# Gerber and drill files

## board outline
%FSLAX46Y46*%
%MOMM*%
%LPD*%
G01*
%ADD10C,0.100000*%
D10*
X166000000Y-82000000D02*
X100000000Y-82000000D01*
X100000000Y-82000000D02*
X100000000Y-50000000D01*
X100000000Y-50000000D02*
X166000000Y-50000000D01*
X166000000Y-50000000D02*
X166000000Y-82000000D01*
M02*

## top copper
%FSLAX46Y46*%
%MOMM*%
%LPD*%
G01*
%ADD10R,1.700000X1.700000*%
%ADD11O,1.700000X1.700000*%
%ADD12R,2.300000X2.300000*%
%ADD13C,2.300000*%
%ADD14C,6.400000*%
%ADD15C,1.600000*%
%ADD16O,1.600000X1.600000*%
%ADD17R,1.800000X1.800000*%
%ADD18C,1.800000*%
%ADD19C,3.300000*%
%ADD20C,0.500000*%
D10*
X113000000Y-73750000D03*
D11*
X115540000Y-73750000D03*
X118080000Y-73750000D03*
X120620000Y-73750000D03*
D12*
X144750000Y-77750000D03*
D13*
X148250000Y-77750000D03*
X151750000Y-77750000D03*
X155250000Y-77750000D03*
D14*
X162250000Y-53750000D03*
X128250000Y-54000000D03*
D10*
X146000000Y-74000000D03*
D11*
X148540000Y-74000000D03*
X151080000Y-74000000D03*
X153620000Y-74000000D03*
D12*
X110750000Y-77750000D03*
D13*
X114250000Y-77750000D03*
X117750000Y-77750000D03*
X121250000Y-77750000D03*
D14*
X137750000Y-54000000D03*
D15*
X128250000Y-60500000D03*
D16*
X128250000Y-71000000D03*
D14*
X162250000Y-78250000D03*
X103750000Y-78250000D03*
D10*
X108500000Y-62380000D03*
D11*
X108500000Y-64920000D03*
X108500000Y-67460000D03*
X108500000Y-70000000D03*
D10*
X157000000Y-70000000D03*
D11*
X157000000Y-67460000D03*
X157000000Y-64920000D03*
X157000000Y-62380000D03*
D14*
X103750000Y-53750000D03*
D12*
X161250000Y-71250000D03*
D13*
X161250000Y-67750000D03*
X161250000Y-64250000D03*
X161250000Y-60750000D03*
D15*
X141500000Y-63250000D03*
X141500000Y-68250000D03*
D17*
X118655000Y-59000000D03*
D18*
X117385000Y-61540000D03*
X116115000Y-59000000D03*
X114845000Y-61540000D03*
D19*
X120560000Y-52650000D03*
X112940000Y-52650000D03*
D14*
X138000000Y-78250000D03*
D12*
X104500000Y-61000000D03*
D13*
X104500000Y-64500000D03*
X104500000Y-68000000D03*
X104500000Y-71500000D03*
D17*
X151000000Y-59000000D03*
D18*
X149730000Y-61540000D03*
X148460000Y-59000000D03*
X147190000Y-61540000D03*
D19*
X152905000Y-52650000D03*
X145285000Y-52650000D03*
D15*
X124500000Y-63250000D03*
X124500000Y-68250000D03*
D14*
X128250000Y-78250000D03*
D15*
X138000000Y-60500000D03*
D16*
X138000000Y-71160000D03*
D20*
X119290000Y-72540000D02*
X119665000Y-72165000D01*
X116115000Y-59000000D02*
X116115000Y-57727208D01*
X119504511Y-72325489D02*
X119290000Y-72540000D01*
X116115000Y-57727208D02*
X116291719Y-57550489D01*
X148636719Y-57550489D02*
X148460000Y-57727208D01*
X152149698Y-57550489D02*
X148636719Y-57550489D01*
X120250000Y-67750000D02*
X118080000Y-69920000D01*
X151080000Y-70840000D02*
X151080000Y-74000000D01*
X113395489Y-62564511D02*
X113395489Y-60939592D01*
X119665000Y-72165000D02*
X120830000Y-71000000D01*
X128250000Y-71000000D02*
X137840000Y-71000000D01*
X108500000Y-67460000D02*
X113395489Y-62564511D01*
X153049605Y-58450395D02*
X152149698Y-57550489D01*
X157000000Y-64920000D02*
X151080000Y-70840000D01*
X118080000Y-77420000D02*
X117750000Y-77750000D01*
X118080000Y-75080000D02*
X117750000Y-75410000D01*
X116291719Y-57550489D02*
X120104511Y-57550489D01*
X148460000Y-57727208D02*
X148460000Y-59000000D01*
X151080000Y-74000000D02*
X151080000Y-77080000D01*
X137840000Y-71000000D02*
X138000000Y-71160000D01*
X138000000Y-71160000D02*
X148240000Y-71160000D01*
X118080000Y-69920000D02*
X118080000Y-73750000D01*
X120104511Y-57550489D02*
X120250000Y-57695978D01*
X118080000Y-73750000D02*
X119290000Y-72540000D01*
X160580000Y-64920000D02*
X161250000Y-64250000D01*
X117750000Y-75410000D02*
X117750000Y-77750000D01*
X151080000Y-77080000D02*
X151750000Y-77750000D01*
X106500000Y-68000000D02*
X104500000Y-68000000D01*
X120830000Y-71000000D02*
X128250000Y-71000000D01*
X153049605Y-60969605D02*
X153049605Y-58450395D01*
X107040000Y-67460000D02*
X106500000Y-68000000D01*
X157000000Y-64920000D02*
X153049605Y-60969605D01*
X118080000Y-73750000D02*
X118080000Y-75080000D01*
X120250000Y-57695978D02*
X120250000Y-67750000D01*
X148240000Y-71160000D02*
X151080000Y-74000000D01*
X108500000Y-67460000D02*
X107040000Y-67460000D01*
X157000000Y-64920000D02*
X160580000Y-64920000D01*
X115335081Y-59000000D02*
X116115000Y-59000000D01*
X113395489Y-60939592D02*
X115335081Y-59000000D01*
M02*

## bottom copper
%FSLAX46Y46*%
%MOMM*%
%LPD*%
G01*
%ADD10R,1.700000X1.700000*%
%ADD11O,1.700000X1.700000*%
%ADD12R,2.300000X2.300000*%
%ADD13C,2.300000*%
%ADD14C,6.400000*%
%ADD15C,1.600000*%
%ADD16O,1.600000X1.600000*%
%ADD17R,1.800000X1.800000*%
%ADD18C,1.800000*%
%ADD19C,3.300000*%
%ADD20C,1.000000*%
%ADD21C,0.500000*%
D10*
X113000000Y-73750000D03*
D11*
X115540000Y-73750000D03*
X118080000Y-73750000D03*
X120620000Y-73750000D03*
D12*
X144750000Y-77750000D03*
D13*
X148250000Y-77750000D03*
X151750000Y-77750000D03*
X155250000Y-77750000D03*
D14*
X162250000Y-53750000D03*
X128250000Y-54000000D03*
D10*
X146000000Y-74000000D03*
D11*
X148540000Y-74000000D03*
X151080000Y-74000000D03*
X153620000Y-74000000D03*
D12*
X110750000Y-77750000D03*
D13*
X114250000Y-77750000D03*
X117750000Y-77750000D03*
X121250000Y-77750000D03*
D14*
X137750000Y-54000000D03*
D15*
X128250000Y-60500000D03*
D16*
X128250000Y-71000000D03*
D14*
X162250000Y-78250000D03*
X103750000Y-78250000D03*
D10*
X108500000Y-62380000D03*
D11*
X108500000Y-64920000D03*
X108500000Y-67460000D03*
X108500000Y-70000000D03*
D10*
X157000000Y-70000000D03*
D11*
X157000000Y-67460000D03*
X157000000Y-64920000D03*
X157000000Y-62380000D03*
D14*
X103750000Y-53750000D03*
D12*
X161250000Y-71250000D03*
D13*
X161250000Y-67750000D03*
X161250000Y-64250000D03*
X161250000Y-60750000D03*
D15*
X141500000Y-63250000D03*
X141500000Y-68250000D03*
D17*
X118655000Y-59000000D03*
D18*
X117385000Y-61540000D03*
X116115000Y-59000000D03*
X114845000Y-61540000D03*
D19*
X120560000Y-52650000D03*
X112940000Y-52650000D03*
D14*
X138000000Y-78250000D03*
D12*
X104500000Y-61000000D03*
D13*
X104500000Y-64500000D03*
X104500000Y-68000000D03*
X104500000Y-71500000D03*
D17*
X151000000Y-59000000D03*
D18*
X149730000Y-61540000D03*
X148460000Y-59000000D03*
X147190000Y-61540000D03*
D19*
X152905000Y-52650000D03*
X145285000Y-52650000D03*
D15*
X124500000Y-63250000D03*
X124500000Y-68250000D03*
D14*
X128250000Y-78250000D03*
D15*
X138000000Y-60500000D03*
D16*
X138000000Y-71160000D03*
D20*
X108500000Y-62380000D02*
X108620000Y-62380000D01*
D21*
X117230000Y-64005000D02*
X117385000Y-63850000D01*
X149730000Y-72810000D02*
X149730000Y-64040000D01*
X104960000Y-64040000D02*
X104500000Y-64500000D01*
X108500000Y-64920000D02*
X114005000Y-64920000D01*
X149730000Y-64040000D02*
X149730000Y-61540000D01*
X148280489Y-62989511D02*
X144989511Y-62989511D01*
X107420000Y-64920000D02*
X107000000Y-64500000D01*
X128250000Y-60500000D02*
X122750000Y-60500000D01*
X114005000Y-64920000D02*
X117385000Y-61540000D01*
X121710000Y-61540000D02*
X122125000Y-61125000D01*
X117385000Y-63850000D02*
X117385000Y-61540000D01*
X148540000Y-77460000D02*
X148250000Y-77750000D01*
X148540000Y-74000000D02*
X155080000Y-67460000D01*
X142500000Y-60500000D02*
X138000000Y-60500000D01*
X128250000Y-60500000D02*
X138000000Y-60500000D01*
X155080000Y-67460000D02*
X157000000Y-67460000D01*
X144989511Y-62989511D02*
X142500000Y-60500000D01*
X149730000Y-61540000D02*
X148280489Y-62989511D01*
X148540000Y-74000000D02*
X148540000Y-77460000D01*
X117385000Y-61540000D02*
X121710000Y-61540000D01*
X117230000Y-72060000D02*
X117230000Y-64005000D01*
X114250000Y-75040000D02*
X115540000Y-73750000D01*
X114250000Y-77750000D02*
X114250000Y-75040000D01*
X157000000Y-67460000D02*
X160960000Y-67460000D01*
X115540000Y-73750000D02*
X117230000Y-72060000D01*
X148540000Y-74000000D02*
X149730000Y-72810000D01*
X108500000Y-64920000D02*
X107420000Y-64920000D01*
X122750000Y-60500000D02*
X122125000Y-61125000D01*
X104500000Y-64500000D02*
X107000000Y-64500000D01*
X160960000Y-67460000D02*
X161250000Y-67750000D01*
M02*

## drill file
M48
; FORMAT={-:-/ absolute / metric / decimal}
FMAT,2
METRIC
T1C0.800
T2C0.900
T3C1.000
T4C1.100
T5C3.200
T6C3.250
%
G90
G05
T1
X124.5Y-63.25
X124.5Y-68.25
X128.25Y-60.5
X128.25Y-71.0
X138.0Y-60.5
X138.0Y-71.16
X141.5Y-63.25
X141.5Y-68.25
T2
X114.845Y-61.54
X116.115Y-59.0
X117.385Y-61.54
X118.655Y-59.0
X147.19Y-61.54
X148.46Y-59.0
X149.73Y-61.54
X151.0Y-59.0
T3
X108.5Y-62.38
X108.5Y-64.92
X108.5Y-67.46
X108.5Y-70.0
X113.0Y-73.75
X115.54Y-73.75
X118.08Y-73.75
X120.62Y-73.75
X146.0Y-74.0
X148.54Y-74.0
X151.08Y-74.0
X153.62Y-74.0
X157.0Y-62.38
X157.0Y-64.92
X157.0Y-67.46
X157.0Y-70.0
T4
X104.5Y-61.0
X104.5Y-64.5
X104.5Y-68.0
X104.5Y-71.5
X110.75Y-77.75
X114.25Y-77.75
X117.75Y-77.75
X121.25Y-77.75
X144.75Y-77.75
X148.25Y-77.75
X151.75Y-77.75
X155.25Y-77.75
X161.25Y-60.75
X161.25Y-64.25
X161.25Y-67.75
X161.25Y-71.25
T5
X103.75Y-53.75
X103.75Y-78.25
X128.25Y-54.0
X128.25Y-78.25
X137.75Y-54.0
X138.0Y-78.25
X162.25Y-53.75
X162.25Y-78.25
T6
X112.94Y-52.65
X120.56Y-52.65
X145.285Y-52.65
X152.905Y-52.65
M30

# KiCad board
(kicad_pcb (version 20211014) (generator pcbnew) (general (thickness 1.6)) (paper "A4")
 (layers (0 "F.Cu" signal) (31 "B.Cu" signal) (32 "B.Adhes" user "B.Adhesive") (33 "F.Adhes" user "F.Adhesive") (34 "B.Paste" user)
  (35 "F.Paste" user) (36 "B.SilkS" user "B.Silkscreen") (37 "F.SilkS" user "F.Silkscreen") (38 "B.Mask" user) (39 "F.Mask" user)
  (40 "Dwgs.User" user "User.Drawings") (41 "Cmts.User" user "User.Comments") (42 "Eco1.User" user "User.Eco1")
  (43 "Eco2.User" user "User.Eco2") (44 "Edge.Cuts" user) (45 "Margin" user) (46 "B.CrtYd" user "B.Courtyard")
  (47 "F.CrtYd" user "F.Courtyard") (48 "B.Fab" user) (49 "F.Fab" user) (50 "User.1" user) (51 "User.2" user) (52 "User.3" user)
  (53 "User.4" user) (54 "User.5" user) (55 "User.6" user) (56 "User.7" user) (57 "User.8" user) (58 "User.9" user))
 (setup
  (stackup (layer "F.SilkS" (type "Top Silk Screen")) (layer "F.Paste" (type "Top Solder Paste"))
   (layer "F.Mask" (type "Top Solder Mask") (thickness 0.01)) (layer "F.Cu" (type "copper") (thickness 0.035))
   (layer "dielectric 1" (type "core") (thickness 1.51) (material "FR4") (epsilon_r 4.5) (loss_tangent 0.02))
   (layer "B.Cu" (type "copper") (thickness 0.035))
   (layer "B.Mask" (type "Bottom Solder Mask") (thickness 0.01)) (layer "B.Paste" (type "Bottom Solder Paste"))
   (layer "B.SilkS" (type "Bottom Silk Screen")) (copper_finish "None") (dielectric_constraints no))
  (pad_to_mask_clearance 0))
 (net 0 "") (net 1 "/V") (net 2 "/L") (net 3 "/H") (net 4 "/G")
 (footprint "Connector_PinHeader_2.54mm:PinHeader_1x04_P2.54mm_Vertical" (layer "F.Cu") (at 113 73.75 90)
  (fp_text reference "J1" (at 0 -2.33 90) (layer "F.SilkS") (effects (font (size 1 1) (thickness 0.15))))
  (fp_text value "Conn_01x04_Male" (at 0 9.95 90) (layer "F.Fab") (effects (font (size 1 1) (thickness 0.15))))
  (pad "1" thru_hole rect (at 0 0 90) (size 1.7 1.7) (drill 1) (layers *.Cu *.Mask) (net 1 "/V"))
  (pad "2" thru_hole oval (at 0 2.54 90) (size 1.7 1.7) (drill 1) (layers *.Cu *.Mask) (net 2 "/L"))
  (pad "3" thru_hole oval (at 0 5.08 90) (size 1.7 1.7) (drill 1) (layers *.Cu *.Mask) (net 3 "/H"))
  (pad "4" thru_hole oval (at 0 7.62 90) (size 1.7 1.7) (drill 1) (layers *.Cu *.Mask) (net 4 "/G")))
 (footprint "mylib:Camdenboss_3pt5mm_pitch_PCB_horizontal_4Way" (layer "F.Cu") (at 142.3 76.25)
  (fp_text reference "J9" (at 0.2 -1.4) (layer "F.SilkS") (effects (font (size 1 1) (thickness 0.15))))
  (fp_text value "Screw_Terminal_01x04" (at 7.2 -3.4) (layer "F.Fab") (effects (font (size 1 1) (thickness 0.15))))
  (pad "1" thru_hole rect (at 2.45 1.5 270) (size 2.3 2.3) (drill 1.1) (layers *.Cu *.Mask) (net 1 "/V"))
  (pad "2" thru_hole circle (at 5.95 1.5 270) (size 2.3 2.3) (drill 1.1) (layers *.Cu *.Mask) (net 2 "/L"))
  (pad "3" thru_hole circle (at 9.45 1.5 270) (size 2.3 2.3) (drill 1.1) (layers *.Cu *.Mask) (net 3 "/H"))
  (pad "4" thru_hole circle (at 12.95 1.5 270) (size 2.3 2.3) (drill 1.1) (layers *.Cu *.Mask) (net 4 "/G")))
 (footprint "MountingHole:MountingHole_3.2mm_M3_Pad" (layer "F.Cu") (at 162.25 53.75)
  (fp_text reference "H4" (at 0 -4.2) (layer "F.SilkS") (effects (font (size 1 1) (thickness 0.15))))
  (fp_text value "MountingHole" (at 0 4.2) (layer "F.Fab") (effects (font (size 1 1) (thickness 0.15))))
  (pad "1" thru_hole circle (at 0 0) (size 6.4 6.4) (drill 3.2) (layers *.Cu *.Mask)))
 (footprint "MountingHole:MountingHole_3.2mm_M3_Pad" (layer "F.Cu") (at 128.25 54)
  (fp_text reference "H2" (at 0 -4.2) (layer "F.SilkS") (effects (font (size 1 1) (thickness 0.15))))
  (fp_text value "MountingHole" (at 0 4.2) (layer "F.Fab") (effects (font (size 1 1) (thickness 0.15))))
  (pad "1" thru_hole circle (at 0 0) (size 6.4 6.4) (drill 3.2) (layers *.Cu *.Mask)))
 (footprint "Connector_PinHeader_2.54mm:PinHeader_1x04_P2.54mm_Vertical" (layer "F.Cu") (at 146 74 90)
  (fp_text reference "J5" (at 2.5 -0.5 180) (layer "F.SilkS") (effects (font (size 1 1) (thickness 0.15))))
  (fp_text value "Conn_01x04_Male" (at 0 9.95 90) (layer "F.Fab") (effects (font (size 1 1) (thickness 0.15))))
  (pad "1" thru_hole rect (at 0 0 90) (size 1.7 1.7) (drill 1) (layers *.Cu *.Mask) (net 1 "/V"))
  (pad "2" thru_hole oval (at 0 2.54 90) (size 1.7 1.7) (drill 1) (layers *.Cu *.Mask) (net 2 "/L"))
  (pad "3" thru_hole oval (at 0 5.08 90) (size 1.7 1.7) (drill 1) (layers *.Cu *.Mask) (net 3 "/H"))
  (pad "4" thru_hole oval (at 0 7.62 90) (size 1.7 1.7) (drill 1) (layers *.Cu *.Mask) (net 4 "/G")))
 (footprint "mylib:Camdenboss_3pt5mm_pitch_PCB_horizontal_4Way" (layer "F.Cu") (at 108.3 76.25)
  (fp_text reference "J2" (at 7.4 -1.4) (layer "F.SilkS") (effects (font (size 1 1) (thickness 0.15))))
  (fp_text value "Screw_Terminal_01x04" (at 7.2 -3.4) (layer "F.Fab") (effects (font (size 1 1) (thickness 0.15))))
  (pad "1" thru_hole rect (at 2.45 1.5 270) (size 2.3 2.3) (drill 1.1) (layers *.Cu *.Mask) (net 1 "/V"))
  (pad "2" thru_hole circle (at 5.95 1.5 270) (size 2.3 2.3) (drill 1.1) (layers *.Cu *.Mask) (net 2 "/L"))
  (pad "3" thru_hole circle (at 9.45 1.5 270) (size 2.3 2.3) (drill 1.1) (layers *.Cu *.Mask) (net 3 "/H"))
  (pad "4" thru_hole circle (at 12.95 1.5 270) (size 2.3 2.3) (drill 1.1) (layers *.Cu *.Mask) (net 4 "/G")))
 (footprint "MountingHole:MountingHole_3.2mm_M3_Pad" (layer "F.Cu") (at 137.75 54)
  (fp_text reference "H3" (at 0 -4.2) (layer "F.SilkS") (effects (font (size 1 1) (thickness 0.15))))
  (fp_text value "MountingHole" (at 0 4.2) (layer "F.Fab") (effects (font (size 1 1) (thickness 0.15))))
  (pad "1" thru_hole circle (at 0 0) (size 6.4 6.4) (drill 3.2) (layers *.Cu *.Mask)))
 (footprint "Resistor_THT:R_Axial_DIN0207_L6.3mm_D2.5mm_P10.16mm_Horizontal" (layer "F.Cu") (at 128.25 60.84 -90)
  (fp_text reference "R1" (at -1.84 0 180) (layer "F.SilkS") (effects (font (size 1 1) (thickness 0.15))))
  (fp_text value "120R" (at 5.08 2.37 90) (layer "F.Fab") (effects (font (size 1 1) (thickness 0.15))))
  (pad "1" thru_hole circle (at -0.34 0 270) (size 1.6 1.6) (drill 0.8) (layers *.Cu *.Mask) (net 2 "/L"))
  (pad "2" thru_hole oval (at 10.16 0 270) (size 1.6 1.6) (drill 0.8) (layers *.Cu *.Mask) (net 3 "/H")))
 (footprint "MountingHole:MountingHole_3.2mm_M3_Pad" (layer "F.Cu") (at 162.25 78.25)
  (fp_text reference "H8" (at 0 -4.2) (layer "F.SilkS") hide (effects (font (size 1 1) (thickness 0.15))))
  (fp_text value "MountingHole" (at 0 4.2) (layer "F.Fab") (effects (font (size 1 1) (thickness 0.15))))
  (pad "1" thru_hole circle (at 0 0) (size 6.4 6.4) (drill 3.2) (layers *.Cu *.Mask)))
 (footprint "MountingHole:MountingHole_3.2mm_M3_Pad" (layer "F.Cu") (at 103.75 78.25)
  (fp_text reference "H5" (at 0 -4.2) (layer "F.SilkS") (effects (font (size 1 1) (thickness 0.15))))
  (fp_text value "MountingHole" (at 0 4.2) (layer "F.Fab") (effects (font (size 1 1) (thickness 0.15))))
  (pad "1" thru_hole circle (at 0 0) (size 6.4 6.4) (drill 3.2) (layers *.Cu *.Mask)))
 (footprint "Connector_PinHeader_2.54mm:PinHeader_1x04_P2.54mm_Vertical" (layer "F.Cu") (at 108.5 62.38)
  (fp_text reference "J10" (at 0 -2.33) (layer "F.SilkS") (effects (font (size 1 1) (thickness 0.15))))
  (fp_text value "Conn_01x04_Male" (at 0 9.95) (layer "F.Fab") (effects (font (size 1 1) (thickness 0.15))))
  (pad "1" thru_hole rect (at 0 0) (size 1.7 1.7) (drill 1) (layers *.Cu *.Mask) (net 1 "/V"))
  (pad "2" thru_hole oval (at 0 2.54) (size 1.7 1.7) (drill 1) (layers *.Cu *.Mask) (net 2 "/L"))
  (pad "3" thru_hole oval (at 0 5.08) (size 1.7 1.7) (drill 1) (layers *.Cu *.Mask) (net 3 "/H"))
  (pad "4" thru_hole oval (at 0 7.62) (size 1.7 1.7) (drill 1) (layers *.Cu *.Mask) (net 4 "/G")))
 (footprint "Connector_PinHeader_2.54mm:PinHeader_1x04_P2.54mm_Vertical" (layer "F.Cu") (at 157 70 180)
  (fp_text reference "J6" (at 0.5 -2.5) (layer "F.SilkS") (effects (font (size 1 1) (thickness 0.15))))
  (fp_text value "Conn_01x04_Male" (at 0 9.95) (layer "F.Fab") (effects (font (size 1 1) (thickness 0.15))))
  (pad "1" thru_hole rect (at 0 0 180) (size 1.7 1.7) (drill 1) (layers *.Cu *.Mask) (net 1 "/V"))
  (pad "2" thru_hole oval (at 0 2.54 180) (size 1.7 1.7) (drill 1) (layers *.Cu *.Mask) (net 2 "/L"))
  (pad "3" thru_hole oval (at 0 5.08 180) (size 1.7 1.7) (drill 1) (layers *.Cu *.Mask) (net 3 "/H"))
  (pad "4" thru_hole oval (at 0 7.62 180) (size 1.7 1.7) (drill 1) (layers *.Cu *.Mask) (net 4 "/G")))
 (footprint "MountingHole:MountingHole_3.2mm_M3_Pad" (layer "F.Cu") (at 103.75 53.75)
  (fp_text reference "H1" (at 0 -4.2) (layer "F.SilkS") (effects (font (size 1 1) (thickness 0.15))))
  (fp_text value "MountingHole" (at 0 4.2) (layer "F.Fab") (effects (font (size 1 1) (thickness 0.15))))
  (pad "1" thru_hole circle (at 0 0) (size 6.4 6.4) (drill 3.2) (layers *.Cu *.Mask)))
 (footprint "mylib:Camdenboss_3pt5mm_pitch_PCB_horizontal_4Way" (layer "F.Cu") (at 159.75 73.7 90)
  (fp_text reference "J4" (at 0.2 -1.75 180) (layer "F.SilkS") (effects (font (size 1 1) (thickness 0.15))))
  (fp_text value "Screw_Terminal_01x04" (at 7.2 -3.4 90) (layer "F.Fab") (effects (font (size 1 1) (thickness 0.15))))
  (pad "1" thru_hole rect (at 2.45 1.5) (size 2.3 2.3) (drill 1.1) (layers *.Cu *.Mask) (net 1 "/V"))
  (pad "2" thru_hole circle (at 5.95 1.5) (size 2.3 2.3) (drill 1.1) (layers *.Cu *.Mask) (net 2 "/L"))
  (pad "3" thru_hole circle (at 9.45 1.5) (size 2.3 2.3) (drill 1.1) (layers *.Cu *.Mask) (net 3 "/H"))
  (pad "4" thru_hole circle (at 12.95 1.5) (size 2.3 2.3) (drill 1.1) (layers *.Cu *.Mask) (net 4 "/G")))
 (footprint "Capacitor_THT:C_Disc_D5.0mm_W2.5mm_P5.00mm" (layer "F.Cu") (at 141.5 63.25 -90)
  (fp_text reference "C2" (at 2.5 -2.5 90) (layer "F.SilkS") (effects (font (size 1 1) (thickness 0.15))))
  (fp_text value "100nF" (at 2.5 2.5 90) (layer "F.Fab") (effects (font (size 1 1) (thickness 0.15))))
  (pad "1" thru_hole circle (at 0 0 270) (size 1.6 1.6) (drill 0.8) (layers *.Cu *.Mask) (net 1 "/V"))
  (pad "2" thru_hole circle (at 5 0 270) (size 1.6 1.6) (drill 0.8) (layers *.Cu *.Mask) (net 4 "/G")))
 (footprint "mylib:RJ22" (layer "F.Cu") (at 116.75 61.54 180)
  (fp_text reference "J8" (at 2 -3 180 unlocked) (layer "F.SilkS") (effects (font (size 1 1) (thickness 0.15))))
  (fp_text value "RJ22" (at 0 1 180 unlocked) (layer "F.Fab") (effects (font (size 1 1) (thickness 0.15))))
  (pad "1" thru_hole rect (at -1.905 2.54 180) (size 1.8 1.8) (drill 0.9) (layers *.Cu *.Mask) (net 1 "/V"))
  (pad "2" thru_hole circle (at -0.635 0 180) (size 1.8 1.8) (drill 0.9) (layers *.Cu *.Mask) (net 2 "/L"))
  (pad "3" thru_hole circle (at 0.635 2.54 180) (size 1.8 1.8) (drill 0.9) (layers *.Cu *.Mask) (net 3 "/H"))
  (pad "4" thru_hole circle (at 1.905 0 180) (size 1.8 1.8) (drill 0.9) (layers *.Cu *.Mask) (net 4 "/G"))
  (pad "5" thru_hole circle (at -3.81 8.89 180) (size 3.3 3.3) (drill 3.25) (layers *.Cu *.Mask))
  (pad "6" thru_hole circle (at 3.81 8.89 180) (size 3.3 3.3) (drill 3.25) (layers *.Cu *.Mask)))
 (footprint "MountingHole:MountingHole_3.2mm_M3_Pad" (layer "F.Cu") (at 138 78.25)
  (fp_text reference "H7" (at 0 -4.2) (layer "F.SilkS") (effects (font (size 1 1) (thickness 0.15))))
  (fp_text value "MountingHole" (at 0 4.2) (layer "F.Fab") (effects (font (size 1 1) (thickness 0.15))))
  (pad "1" thru_hole circle (at 0 0) (size 6.4 6.4) (drill 3.2) (layers *.Cu *.Mask)))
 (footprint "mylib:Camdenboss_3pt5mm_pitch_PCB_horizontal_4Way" (layer "F.Cu") (at 106 58.55 -90)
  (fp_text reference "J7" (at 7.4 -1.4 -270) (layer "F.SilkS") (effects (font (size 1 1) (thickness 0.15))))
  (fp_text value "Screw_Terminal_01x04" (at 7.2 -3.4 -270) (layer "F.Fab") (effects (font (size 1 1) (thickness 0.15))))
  (pad "1" thru_hole rect (at 2.45 1.5 180) (size 2.3 2.3) (drill 1.1) (layers *.Cu *.Mask) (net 1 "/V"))
  (pad "2" thru_hole circle (at 5.95 1.5 180) (size 2.3 2.3) (drill 1.1) (layers *.Cu *.Mask) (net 2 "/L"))
  (pad "3" thru_hole circle (at 9.45 1.5 180) (size 2.3 2.3) (drill 1.1) (layers *.Cu *.Mask) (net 3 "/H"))
  (pad "4" thru_hole circle (at 12.95 1.5 180) (size 2.3 2.3) (drill 1.1) (layers *.Cu *.Mask) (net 4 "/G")))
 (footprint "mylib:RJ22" (layer "F.Cu") (at 149.095 61.54 180)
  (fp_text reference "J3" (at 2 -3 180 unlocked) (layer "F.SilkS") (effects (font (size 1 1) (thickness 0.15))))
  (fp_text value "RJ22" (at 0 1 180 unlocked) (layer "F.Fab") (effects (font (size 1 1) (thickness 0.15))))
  (pad "1" thru_hole rect (at -1.905 2.54 180) (size 1.8 1.8) (drill 0.9) (layers *.Cu *.Mask) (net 1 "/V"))
  (pad "2" thru_hole circle (at -0.635 0 180) (size 1.8 1.8) (drill 0.9) (layers *.Cu *.Mask) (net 2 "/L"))
  (pad "3" thru_hole circle (at 0.635 2.54 180) (size 1.8 1.8) (drill 0.9) (layers *.Cu *.Mask) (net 3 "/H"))
  (pad "4" thru_hole circle (at 1.905 0 180) (size 1.8 1.8) (drill 0.9) (layers *.Cu *.Mask) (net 4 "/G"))
  (pad "5" thru_hole circle (at -3.81 8.89 180) (size 3.3 3.3) (drill 3.25) (layers *.Cu *.Mask))
  (pad "6" thru_hole circle (at 3.81 8.89 180) (size 3.3 3.3) (drill 3.25) (layers *.Cu *.Mask)))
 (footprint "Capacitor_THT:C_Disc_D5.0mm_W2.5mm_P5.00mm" (layer "F.Cu") (at 124.5 63.25 -90)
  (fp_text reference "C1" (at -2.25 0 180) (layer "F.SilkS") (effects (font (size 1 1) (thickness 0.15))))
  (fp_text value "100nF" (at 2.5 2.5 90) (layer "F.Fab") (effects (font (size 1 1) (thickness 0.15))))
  (pad "1" thru_hole circle (at 0 0 270) (size 1.6 1.6) (drill 0.8) (layers *.Cu *.Mask) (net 1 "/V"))
  (pad "2" thru_hole circle (at 5 0 270) (size 1.6 1.6) (drill 0.8) (layers *.Cu *.Mask) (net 4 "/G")))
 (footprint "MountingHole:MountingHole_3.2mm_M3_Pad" (layer "F.Cu") (at 128.25 78.25)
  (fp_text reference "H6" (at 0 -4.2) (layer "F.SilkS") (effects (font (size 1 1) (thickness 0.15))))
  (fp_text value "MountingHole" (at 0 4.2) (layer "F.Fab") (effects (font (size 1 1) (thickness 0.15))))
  (pad "1" thru_hole circle (at 0 0) (size 6.4 6.4) (drill 3.2) (layers *.Cu *.Mask)))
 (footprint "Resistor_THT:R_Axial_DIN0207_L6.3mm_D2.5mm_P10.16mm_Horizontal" (layer "F.Cu") (at 138 61 -90)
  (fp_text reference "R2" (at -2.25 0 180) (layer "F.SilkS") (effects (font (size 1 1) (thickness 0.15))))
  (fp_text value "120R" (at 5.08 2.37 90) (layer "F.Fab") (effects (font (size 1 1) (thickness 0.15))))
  (pad "1" thru_hole circle (at -0.5 0 270) (size 1.6 1.6) (drill 0.8) (layers *.Cu *.Mask) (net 2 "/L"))
  (pad "2" thru_hole oval (at 10.16 0 270) (size 1.6 1.6) (drill 0.8) (layers *.Cu *.Mask) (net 3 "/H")))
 (gr_line (start 166 82) (end 100 82) (layer "Edge.Cuts") (width 0.1))
 (gr_line (start 100 82) (end 100 50) (layer "Edge.Cuts") (width 0.1))
 (gr_line (start 100 50) (end 166 50) (layer "Edge.Cuts") (width 0.1))
 (gr_line (start 166 50) (end 166 82) (layer "Edge.Cuts") (width 0.1))
 (segment (start 108.5 62.38) (end 108.62 62.38) (width 1) (layer "B.Cu") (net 1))
 (segment (start 117.23 64.005) (end 117.385 63.85) (width 0.5) (layer "B.Cu") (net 2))
 (segment (start 149.73 72.81) (end 149.73 64.04) (width 0.5) (layer "B.Cu") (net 2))
 (segment (start 104.96 64.04) (end 104.5 64.5) (width 0.5) (layer "B.Cu") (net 2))
 (segment (start 108.5 64.92) (end 114.005 64.92) (width 0.5) (layer "B.Cu") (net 2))
 (segment (start 149.73 64.04) (end 149.73 61.54) (width 0.5) (layer "B.Cu") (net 2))
 (segment (start 148.280489 62.989511) (end 144.989511 62.989511) (width 0.5) (layer "B.Cu") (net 2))
 (segment (start 107.42 64.92) (end 107 64.5) (width 0.5) (layer "B.Cu") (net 2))
 (segment (start 128.25 60.5) (end 122.75 60.5) (width 0.5) (layer "B.Cu") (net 2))
 (segment (start 114.005 64.92) (end 117.385 61.54) (width 0.5) (layer "B.Cu") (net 2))
 (segment (start 121.71 61.54) (end 122.125 61.125) (width 0.5) (layer "B.Cu") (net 2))
 (segment (start 117.385 63.85) (end 117.385 61.54) (width 0.5) (layer "B.Cu") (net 2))
 (segment (start 148.54 77.46) (end 148.25 77.75) (width 0.5) (layer "B.Cu") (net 2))
 (segment (start 148.54 74) (end 155.08 67.46) (width 0.5) (layer "B.Cu") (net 2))
 (segment (start 142.5 60.5) (end 138 60.5) (width 0.5) (layer "B.Cu") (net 2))
 (segment (start 128.25 60.5) (end 138 60.5) (width 0.5) (layer "B.Cu") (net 2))
 (segment (start 155.08 67.46) (end 157 67.46) (width 0.5) (layer "B.Cu") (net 2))
 (segment (start 144.989511 62.989511) (end 142.5 60.5) (width 0.5) (layer "B.Cu") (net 2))
 (segment (start 149.73 61.54) (end 148.280489 62.989511) (width 0.5) (layer "B.Cu") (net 2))
 (segment (start 148.54 74) (end 148.54 77.46) (width 0.5) (layer "B.Cu") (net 2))
 (segment (start 117.385 61.54) (end 121.71 61.54) (width 0.5) (layer "B.Cu") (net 2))
 (segment (start 117.23 72.06) (end 117.23 64.005) (width 0.5) (layer "B.Cu") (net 2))
 (segment (start 114.25 75.04) (end 115.54 73.75) (width 0.5) (layer "B.Cu") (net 2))
 (segment (start 114.25 77.75) (end 114.25 75.04) (width 0.5) (layer "B.Cu") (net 2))
 (segment (start 157 67.46) (end 160.96 67.46) (width 0.5) (layer "B.Cu") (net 2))
 (segment (start 115.54 73.75) (end 117.23 72.06) (width 0.5) (layer "B.Cu") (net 2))
 (segment (start 148.54 74) (end 149.73 72.81) (width 0.5) (layer "B.Cu") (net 2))
 (segment (start 108.5 64.92) (end 107.42 64.92) (width 0.5) (layer "B.Cu") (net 2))
 (segment (start 122.75 60.5) (end 122.125 61.125) (width 0.5) (layer "B.Cu") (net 2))
 (segment (start 104.5 64.5) (end 107 64.5) (width 0.5) (layer "B.Cu") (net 2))
 (segment (start 160.96 67.46) (end 161.25 67.75) (width 0.5) (layer "B.Cu") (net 2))
 (segment (start 119.29 72.54) (end 119.665 72.165) (width 0.5) (layer "F.Cu") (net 3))
 (segment (start 116.115 59) (end 116.115 57.727208) (width 0.5) (layer "F.Cu") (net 3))
 (segment (start 119.504511 72.325489) (end 119.29 72.54) (width 0.5) (layer "F.Cu") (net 3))
 (segment (start 116.115 57.727208) (end 116.291719 57.550489) (width 0.5) (layer "F.Cu") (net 3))
 (segment (start 148.636719 57.550489) (end 148.46 57.727208) (width 0.5) (layer "F.Cu") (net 3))
 (segment (start 152.149698 57.550489) (end 148.636719 57.550489) (width 0.5) (layer "F.Cu") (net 3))
 (segment (start 120.25 67.75) (end 118.08 69.92) (width 0.5) (layer "F.Cu") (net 3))
 (segment (start 151.08 70.84) (end 151.08 74) (width 0.5) (layer "F.Cu") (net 3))
 (segment (start 113.395489 62.564511) (end 113.395489 60.939592) (width 0.5) (layer "F.Cu") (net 3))
 (segment (start 119.665 72.165) (end 120.83 71) (width 0.5) (layer "F.Cu") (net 3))
 (segment (start 128.25 71) (end 137.84 71) (width 0.5) (layer "F.Cu") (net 3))
 (segment (start 108.5 67.46) (end 113.395489 62.564511) (width 0.5) (layer "F.Cu") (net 3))
 (segment (start 153.049605 58.450395) (end 152.149698 57.550489) (width 0.5) (layer "F.Cu") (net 3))
 (segment (start 157 64.92) (end 151.08 70.84) (width 0.5) (layer "F.Cu") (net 3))
 (segment (start 118.08 77.42) (end 117.75 77.75) (width 0.5) (layer "F.Cu") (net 3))
 (segment (start 118.08 75.08) (end 117.75 75.41) (width 0.5) (layer "F.Cu") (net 3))
 (segment (start 116.291719 57.550489) (end 120.104511 57.550489) (width 0.5) (layer "F.Cu") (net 3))
 (segment (start 148.46 57.727208) (end 148.46 59) (width 0.5) (layer "F.Cu") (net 3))
 (segment (start 151.08 74) (end 151.08 77.08) (width 0.5) (layer "F.Cu") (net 3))
 (segment (start 137.84 71) (end 138 71.16) (width 0.5) (layer "F.Cu") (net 3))
 (segment (start 138 71.16) (end 148.24 71.16) (width 0.5) (layer "F.Cu") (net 3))
 (segment (start 118.08 69.92) (end 118.08 73.75) (width 0.5) (layer "F.Cu") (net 3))
 (segment (start 120.104511 57.550489) (end 120.25 57.695978) (width 0.5) (layer "F.Cu") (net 3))
 (segment (start 118.08 73.75) (end 119.29 72.54) (width 0.5) (layer "F.Cu") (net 3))
 (segment (start 160.58 64.92) (end 161.25 64.25) (width 0.5) (layer "F.Cu") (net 3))
 (segment (start 117.75 75.41) (end 117.75 77.75) (width 0.5) (layer "F.Cu") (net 3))
 (segment (start 151.08 77.08) (end 151.75 77.75) (width 0.5) (layer "F.Cu") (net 3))
 (segment (start 106.5 68) (end 104.5 68) (width 0.5) (layer "F.Cu") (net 3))
 (segment (start 120.83 71) (end 128.25 71) (width 0.5) (layer "F.Cu") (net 3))
 (segment (start 153.049605 60.969605) (end 153.049605 58.450395) (width 0.5) (layer "F.Cu") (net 3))
 (segment (start 107.04 67.46) (end 106.5 68) (width 0.5) (layer "F.Cu") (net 3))
 (segment (start 157 64.92) (end 153.049605 60.969605) (width 0.5) (layer "F.Cu") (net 3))
 (segment (start 118.08 73.75) (end 118.08 75.08) (width 0.5) (layer "F.Cu") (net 3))
 (segment (start 120.25 57.695978) (end 120.25 67.75) (width 0.5) (layer "F.Cu") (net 3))
 (segment (start 148.24 71.16) (end 151.08 74) (width 0.5) (layer "F.Cu") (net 3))
 (segment (start 108.5 67.46) (end 107.04 67.46) (width 0.5) (layer "F.Cu") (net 3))
 (segment (start 157 64.92) (end 160.58 64.92) (width 0.5) (layer "F.Cu") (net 3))
 (segment (start 115.335081 59) (end 116.115 59) (width 0.5) (layer "F.Cu") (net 3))
 (segment (start 113.395489 60.939592) (end 115.335081 59) (width 0.5) (layer "F.Cu") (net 3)))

